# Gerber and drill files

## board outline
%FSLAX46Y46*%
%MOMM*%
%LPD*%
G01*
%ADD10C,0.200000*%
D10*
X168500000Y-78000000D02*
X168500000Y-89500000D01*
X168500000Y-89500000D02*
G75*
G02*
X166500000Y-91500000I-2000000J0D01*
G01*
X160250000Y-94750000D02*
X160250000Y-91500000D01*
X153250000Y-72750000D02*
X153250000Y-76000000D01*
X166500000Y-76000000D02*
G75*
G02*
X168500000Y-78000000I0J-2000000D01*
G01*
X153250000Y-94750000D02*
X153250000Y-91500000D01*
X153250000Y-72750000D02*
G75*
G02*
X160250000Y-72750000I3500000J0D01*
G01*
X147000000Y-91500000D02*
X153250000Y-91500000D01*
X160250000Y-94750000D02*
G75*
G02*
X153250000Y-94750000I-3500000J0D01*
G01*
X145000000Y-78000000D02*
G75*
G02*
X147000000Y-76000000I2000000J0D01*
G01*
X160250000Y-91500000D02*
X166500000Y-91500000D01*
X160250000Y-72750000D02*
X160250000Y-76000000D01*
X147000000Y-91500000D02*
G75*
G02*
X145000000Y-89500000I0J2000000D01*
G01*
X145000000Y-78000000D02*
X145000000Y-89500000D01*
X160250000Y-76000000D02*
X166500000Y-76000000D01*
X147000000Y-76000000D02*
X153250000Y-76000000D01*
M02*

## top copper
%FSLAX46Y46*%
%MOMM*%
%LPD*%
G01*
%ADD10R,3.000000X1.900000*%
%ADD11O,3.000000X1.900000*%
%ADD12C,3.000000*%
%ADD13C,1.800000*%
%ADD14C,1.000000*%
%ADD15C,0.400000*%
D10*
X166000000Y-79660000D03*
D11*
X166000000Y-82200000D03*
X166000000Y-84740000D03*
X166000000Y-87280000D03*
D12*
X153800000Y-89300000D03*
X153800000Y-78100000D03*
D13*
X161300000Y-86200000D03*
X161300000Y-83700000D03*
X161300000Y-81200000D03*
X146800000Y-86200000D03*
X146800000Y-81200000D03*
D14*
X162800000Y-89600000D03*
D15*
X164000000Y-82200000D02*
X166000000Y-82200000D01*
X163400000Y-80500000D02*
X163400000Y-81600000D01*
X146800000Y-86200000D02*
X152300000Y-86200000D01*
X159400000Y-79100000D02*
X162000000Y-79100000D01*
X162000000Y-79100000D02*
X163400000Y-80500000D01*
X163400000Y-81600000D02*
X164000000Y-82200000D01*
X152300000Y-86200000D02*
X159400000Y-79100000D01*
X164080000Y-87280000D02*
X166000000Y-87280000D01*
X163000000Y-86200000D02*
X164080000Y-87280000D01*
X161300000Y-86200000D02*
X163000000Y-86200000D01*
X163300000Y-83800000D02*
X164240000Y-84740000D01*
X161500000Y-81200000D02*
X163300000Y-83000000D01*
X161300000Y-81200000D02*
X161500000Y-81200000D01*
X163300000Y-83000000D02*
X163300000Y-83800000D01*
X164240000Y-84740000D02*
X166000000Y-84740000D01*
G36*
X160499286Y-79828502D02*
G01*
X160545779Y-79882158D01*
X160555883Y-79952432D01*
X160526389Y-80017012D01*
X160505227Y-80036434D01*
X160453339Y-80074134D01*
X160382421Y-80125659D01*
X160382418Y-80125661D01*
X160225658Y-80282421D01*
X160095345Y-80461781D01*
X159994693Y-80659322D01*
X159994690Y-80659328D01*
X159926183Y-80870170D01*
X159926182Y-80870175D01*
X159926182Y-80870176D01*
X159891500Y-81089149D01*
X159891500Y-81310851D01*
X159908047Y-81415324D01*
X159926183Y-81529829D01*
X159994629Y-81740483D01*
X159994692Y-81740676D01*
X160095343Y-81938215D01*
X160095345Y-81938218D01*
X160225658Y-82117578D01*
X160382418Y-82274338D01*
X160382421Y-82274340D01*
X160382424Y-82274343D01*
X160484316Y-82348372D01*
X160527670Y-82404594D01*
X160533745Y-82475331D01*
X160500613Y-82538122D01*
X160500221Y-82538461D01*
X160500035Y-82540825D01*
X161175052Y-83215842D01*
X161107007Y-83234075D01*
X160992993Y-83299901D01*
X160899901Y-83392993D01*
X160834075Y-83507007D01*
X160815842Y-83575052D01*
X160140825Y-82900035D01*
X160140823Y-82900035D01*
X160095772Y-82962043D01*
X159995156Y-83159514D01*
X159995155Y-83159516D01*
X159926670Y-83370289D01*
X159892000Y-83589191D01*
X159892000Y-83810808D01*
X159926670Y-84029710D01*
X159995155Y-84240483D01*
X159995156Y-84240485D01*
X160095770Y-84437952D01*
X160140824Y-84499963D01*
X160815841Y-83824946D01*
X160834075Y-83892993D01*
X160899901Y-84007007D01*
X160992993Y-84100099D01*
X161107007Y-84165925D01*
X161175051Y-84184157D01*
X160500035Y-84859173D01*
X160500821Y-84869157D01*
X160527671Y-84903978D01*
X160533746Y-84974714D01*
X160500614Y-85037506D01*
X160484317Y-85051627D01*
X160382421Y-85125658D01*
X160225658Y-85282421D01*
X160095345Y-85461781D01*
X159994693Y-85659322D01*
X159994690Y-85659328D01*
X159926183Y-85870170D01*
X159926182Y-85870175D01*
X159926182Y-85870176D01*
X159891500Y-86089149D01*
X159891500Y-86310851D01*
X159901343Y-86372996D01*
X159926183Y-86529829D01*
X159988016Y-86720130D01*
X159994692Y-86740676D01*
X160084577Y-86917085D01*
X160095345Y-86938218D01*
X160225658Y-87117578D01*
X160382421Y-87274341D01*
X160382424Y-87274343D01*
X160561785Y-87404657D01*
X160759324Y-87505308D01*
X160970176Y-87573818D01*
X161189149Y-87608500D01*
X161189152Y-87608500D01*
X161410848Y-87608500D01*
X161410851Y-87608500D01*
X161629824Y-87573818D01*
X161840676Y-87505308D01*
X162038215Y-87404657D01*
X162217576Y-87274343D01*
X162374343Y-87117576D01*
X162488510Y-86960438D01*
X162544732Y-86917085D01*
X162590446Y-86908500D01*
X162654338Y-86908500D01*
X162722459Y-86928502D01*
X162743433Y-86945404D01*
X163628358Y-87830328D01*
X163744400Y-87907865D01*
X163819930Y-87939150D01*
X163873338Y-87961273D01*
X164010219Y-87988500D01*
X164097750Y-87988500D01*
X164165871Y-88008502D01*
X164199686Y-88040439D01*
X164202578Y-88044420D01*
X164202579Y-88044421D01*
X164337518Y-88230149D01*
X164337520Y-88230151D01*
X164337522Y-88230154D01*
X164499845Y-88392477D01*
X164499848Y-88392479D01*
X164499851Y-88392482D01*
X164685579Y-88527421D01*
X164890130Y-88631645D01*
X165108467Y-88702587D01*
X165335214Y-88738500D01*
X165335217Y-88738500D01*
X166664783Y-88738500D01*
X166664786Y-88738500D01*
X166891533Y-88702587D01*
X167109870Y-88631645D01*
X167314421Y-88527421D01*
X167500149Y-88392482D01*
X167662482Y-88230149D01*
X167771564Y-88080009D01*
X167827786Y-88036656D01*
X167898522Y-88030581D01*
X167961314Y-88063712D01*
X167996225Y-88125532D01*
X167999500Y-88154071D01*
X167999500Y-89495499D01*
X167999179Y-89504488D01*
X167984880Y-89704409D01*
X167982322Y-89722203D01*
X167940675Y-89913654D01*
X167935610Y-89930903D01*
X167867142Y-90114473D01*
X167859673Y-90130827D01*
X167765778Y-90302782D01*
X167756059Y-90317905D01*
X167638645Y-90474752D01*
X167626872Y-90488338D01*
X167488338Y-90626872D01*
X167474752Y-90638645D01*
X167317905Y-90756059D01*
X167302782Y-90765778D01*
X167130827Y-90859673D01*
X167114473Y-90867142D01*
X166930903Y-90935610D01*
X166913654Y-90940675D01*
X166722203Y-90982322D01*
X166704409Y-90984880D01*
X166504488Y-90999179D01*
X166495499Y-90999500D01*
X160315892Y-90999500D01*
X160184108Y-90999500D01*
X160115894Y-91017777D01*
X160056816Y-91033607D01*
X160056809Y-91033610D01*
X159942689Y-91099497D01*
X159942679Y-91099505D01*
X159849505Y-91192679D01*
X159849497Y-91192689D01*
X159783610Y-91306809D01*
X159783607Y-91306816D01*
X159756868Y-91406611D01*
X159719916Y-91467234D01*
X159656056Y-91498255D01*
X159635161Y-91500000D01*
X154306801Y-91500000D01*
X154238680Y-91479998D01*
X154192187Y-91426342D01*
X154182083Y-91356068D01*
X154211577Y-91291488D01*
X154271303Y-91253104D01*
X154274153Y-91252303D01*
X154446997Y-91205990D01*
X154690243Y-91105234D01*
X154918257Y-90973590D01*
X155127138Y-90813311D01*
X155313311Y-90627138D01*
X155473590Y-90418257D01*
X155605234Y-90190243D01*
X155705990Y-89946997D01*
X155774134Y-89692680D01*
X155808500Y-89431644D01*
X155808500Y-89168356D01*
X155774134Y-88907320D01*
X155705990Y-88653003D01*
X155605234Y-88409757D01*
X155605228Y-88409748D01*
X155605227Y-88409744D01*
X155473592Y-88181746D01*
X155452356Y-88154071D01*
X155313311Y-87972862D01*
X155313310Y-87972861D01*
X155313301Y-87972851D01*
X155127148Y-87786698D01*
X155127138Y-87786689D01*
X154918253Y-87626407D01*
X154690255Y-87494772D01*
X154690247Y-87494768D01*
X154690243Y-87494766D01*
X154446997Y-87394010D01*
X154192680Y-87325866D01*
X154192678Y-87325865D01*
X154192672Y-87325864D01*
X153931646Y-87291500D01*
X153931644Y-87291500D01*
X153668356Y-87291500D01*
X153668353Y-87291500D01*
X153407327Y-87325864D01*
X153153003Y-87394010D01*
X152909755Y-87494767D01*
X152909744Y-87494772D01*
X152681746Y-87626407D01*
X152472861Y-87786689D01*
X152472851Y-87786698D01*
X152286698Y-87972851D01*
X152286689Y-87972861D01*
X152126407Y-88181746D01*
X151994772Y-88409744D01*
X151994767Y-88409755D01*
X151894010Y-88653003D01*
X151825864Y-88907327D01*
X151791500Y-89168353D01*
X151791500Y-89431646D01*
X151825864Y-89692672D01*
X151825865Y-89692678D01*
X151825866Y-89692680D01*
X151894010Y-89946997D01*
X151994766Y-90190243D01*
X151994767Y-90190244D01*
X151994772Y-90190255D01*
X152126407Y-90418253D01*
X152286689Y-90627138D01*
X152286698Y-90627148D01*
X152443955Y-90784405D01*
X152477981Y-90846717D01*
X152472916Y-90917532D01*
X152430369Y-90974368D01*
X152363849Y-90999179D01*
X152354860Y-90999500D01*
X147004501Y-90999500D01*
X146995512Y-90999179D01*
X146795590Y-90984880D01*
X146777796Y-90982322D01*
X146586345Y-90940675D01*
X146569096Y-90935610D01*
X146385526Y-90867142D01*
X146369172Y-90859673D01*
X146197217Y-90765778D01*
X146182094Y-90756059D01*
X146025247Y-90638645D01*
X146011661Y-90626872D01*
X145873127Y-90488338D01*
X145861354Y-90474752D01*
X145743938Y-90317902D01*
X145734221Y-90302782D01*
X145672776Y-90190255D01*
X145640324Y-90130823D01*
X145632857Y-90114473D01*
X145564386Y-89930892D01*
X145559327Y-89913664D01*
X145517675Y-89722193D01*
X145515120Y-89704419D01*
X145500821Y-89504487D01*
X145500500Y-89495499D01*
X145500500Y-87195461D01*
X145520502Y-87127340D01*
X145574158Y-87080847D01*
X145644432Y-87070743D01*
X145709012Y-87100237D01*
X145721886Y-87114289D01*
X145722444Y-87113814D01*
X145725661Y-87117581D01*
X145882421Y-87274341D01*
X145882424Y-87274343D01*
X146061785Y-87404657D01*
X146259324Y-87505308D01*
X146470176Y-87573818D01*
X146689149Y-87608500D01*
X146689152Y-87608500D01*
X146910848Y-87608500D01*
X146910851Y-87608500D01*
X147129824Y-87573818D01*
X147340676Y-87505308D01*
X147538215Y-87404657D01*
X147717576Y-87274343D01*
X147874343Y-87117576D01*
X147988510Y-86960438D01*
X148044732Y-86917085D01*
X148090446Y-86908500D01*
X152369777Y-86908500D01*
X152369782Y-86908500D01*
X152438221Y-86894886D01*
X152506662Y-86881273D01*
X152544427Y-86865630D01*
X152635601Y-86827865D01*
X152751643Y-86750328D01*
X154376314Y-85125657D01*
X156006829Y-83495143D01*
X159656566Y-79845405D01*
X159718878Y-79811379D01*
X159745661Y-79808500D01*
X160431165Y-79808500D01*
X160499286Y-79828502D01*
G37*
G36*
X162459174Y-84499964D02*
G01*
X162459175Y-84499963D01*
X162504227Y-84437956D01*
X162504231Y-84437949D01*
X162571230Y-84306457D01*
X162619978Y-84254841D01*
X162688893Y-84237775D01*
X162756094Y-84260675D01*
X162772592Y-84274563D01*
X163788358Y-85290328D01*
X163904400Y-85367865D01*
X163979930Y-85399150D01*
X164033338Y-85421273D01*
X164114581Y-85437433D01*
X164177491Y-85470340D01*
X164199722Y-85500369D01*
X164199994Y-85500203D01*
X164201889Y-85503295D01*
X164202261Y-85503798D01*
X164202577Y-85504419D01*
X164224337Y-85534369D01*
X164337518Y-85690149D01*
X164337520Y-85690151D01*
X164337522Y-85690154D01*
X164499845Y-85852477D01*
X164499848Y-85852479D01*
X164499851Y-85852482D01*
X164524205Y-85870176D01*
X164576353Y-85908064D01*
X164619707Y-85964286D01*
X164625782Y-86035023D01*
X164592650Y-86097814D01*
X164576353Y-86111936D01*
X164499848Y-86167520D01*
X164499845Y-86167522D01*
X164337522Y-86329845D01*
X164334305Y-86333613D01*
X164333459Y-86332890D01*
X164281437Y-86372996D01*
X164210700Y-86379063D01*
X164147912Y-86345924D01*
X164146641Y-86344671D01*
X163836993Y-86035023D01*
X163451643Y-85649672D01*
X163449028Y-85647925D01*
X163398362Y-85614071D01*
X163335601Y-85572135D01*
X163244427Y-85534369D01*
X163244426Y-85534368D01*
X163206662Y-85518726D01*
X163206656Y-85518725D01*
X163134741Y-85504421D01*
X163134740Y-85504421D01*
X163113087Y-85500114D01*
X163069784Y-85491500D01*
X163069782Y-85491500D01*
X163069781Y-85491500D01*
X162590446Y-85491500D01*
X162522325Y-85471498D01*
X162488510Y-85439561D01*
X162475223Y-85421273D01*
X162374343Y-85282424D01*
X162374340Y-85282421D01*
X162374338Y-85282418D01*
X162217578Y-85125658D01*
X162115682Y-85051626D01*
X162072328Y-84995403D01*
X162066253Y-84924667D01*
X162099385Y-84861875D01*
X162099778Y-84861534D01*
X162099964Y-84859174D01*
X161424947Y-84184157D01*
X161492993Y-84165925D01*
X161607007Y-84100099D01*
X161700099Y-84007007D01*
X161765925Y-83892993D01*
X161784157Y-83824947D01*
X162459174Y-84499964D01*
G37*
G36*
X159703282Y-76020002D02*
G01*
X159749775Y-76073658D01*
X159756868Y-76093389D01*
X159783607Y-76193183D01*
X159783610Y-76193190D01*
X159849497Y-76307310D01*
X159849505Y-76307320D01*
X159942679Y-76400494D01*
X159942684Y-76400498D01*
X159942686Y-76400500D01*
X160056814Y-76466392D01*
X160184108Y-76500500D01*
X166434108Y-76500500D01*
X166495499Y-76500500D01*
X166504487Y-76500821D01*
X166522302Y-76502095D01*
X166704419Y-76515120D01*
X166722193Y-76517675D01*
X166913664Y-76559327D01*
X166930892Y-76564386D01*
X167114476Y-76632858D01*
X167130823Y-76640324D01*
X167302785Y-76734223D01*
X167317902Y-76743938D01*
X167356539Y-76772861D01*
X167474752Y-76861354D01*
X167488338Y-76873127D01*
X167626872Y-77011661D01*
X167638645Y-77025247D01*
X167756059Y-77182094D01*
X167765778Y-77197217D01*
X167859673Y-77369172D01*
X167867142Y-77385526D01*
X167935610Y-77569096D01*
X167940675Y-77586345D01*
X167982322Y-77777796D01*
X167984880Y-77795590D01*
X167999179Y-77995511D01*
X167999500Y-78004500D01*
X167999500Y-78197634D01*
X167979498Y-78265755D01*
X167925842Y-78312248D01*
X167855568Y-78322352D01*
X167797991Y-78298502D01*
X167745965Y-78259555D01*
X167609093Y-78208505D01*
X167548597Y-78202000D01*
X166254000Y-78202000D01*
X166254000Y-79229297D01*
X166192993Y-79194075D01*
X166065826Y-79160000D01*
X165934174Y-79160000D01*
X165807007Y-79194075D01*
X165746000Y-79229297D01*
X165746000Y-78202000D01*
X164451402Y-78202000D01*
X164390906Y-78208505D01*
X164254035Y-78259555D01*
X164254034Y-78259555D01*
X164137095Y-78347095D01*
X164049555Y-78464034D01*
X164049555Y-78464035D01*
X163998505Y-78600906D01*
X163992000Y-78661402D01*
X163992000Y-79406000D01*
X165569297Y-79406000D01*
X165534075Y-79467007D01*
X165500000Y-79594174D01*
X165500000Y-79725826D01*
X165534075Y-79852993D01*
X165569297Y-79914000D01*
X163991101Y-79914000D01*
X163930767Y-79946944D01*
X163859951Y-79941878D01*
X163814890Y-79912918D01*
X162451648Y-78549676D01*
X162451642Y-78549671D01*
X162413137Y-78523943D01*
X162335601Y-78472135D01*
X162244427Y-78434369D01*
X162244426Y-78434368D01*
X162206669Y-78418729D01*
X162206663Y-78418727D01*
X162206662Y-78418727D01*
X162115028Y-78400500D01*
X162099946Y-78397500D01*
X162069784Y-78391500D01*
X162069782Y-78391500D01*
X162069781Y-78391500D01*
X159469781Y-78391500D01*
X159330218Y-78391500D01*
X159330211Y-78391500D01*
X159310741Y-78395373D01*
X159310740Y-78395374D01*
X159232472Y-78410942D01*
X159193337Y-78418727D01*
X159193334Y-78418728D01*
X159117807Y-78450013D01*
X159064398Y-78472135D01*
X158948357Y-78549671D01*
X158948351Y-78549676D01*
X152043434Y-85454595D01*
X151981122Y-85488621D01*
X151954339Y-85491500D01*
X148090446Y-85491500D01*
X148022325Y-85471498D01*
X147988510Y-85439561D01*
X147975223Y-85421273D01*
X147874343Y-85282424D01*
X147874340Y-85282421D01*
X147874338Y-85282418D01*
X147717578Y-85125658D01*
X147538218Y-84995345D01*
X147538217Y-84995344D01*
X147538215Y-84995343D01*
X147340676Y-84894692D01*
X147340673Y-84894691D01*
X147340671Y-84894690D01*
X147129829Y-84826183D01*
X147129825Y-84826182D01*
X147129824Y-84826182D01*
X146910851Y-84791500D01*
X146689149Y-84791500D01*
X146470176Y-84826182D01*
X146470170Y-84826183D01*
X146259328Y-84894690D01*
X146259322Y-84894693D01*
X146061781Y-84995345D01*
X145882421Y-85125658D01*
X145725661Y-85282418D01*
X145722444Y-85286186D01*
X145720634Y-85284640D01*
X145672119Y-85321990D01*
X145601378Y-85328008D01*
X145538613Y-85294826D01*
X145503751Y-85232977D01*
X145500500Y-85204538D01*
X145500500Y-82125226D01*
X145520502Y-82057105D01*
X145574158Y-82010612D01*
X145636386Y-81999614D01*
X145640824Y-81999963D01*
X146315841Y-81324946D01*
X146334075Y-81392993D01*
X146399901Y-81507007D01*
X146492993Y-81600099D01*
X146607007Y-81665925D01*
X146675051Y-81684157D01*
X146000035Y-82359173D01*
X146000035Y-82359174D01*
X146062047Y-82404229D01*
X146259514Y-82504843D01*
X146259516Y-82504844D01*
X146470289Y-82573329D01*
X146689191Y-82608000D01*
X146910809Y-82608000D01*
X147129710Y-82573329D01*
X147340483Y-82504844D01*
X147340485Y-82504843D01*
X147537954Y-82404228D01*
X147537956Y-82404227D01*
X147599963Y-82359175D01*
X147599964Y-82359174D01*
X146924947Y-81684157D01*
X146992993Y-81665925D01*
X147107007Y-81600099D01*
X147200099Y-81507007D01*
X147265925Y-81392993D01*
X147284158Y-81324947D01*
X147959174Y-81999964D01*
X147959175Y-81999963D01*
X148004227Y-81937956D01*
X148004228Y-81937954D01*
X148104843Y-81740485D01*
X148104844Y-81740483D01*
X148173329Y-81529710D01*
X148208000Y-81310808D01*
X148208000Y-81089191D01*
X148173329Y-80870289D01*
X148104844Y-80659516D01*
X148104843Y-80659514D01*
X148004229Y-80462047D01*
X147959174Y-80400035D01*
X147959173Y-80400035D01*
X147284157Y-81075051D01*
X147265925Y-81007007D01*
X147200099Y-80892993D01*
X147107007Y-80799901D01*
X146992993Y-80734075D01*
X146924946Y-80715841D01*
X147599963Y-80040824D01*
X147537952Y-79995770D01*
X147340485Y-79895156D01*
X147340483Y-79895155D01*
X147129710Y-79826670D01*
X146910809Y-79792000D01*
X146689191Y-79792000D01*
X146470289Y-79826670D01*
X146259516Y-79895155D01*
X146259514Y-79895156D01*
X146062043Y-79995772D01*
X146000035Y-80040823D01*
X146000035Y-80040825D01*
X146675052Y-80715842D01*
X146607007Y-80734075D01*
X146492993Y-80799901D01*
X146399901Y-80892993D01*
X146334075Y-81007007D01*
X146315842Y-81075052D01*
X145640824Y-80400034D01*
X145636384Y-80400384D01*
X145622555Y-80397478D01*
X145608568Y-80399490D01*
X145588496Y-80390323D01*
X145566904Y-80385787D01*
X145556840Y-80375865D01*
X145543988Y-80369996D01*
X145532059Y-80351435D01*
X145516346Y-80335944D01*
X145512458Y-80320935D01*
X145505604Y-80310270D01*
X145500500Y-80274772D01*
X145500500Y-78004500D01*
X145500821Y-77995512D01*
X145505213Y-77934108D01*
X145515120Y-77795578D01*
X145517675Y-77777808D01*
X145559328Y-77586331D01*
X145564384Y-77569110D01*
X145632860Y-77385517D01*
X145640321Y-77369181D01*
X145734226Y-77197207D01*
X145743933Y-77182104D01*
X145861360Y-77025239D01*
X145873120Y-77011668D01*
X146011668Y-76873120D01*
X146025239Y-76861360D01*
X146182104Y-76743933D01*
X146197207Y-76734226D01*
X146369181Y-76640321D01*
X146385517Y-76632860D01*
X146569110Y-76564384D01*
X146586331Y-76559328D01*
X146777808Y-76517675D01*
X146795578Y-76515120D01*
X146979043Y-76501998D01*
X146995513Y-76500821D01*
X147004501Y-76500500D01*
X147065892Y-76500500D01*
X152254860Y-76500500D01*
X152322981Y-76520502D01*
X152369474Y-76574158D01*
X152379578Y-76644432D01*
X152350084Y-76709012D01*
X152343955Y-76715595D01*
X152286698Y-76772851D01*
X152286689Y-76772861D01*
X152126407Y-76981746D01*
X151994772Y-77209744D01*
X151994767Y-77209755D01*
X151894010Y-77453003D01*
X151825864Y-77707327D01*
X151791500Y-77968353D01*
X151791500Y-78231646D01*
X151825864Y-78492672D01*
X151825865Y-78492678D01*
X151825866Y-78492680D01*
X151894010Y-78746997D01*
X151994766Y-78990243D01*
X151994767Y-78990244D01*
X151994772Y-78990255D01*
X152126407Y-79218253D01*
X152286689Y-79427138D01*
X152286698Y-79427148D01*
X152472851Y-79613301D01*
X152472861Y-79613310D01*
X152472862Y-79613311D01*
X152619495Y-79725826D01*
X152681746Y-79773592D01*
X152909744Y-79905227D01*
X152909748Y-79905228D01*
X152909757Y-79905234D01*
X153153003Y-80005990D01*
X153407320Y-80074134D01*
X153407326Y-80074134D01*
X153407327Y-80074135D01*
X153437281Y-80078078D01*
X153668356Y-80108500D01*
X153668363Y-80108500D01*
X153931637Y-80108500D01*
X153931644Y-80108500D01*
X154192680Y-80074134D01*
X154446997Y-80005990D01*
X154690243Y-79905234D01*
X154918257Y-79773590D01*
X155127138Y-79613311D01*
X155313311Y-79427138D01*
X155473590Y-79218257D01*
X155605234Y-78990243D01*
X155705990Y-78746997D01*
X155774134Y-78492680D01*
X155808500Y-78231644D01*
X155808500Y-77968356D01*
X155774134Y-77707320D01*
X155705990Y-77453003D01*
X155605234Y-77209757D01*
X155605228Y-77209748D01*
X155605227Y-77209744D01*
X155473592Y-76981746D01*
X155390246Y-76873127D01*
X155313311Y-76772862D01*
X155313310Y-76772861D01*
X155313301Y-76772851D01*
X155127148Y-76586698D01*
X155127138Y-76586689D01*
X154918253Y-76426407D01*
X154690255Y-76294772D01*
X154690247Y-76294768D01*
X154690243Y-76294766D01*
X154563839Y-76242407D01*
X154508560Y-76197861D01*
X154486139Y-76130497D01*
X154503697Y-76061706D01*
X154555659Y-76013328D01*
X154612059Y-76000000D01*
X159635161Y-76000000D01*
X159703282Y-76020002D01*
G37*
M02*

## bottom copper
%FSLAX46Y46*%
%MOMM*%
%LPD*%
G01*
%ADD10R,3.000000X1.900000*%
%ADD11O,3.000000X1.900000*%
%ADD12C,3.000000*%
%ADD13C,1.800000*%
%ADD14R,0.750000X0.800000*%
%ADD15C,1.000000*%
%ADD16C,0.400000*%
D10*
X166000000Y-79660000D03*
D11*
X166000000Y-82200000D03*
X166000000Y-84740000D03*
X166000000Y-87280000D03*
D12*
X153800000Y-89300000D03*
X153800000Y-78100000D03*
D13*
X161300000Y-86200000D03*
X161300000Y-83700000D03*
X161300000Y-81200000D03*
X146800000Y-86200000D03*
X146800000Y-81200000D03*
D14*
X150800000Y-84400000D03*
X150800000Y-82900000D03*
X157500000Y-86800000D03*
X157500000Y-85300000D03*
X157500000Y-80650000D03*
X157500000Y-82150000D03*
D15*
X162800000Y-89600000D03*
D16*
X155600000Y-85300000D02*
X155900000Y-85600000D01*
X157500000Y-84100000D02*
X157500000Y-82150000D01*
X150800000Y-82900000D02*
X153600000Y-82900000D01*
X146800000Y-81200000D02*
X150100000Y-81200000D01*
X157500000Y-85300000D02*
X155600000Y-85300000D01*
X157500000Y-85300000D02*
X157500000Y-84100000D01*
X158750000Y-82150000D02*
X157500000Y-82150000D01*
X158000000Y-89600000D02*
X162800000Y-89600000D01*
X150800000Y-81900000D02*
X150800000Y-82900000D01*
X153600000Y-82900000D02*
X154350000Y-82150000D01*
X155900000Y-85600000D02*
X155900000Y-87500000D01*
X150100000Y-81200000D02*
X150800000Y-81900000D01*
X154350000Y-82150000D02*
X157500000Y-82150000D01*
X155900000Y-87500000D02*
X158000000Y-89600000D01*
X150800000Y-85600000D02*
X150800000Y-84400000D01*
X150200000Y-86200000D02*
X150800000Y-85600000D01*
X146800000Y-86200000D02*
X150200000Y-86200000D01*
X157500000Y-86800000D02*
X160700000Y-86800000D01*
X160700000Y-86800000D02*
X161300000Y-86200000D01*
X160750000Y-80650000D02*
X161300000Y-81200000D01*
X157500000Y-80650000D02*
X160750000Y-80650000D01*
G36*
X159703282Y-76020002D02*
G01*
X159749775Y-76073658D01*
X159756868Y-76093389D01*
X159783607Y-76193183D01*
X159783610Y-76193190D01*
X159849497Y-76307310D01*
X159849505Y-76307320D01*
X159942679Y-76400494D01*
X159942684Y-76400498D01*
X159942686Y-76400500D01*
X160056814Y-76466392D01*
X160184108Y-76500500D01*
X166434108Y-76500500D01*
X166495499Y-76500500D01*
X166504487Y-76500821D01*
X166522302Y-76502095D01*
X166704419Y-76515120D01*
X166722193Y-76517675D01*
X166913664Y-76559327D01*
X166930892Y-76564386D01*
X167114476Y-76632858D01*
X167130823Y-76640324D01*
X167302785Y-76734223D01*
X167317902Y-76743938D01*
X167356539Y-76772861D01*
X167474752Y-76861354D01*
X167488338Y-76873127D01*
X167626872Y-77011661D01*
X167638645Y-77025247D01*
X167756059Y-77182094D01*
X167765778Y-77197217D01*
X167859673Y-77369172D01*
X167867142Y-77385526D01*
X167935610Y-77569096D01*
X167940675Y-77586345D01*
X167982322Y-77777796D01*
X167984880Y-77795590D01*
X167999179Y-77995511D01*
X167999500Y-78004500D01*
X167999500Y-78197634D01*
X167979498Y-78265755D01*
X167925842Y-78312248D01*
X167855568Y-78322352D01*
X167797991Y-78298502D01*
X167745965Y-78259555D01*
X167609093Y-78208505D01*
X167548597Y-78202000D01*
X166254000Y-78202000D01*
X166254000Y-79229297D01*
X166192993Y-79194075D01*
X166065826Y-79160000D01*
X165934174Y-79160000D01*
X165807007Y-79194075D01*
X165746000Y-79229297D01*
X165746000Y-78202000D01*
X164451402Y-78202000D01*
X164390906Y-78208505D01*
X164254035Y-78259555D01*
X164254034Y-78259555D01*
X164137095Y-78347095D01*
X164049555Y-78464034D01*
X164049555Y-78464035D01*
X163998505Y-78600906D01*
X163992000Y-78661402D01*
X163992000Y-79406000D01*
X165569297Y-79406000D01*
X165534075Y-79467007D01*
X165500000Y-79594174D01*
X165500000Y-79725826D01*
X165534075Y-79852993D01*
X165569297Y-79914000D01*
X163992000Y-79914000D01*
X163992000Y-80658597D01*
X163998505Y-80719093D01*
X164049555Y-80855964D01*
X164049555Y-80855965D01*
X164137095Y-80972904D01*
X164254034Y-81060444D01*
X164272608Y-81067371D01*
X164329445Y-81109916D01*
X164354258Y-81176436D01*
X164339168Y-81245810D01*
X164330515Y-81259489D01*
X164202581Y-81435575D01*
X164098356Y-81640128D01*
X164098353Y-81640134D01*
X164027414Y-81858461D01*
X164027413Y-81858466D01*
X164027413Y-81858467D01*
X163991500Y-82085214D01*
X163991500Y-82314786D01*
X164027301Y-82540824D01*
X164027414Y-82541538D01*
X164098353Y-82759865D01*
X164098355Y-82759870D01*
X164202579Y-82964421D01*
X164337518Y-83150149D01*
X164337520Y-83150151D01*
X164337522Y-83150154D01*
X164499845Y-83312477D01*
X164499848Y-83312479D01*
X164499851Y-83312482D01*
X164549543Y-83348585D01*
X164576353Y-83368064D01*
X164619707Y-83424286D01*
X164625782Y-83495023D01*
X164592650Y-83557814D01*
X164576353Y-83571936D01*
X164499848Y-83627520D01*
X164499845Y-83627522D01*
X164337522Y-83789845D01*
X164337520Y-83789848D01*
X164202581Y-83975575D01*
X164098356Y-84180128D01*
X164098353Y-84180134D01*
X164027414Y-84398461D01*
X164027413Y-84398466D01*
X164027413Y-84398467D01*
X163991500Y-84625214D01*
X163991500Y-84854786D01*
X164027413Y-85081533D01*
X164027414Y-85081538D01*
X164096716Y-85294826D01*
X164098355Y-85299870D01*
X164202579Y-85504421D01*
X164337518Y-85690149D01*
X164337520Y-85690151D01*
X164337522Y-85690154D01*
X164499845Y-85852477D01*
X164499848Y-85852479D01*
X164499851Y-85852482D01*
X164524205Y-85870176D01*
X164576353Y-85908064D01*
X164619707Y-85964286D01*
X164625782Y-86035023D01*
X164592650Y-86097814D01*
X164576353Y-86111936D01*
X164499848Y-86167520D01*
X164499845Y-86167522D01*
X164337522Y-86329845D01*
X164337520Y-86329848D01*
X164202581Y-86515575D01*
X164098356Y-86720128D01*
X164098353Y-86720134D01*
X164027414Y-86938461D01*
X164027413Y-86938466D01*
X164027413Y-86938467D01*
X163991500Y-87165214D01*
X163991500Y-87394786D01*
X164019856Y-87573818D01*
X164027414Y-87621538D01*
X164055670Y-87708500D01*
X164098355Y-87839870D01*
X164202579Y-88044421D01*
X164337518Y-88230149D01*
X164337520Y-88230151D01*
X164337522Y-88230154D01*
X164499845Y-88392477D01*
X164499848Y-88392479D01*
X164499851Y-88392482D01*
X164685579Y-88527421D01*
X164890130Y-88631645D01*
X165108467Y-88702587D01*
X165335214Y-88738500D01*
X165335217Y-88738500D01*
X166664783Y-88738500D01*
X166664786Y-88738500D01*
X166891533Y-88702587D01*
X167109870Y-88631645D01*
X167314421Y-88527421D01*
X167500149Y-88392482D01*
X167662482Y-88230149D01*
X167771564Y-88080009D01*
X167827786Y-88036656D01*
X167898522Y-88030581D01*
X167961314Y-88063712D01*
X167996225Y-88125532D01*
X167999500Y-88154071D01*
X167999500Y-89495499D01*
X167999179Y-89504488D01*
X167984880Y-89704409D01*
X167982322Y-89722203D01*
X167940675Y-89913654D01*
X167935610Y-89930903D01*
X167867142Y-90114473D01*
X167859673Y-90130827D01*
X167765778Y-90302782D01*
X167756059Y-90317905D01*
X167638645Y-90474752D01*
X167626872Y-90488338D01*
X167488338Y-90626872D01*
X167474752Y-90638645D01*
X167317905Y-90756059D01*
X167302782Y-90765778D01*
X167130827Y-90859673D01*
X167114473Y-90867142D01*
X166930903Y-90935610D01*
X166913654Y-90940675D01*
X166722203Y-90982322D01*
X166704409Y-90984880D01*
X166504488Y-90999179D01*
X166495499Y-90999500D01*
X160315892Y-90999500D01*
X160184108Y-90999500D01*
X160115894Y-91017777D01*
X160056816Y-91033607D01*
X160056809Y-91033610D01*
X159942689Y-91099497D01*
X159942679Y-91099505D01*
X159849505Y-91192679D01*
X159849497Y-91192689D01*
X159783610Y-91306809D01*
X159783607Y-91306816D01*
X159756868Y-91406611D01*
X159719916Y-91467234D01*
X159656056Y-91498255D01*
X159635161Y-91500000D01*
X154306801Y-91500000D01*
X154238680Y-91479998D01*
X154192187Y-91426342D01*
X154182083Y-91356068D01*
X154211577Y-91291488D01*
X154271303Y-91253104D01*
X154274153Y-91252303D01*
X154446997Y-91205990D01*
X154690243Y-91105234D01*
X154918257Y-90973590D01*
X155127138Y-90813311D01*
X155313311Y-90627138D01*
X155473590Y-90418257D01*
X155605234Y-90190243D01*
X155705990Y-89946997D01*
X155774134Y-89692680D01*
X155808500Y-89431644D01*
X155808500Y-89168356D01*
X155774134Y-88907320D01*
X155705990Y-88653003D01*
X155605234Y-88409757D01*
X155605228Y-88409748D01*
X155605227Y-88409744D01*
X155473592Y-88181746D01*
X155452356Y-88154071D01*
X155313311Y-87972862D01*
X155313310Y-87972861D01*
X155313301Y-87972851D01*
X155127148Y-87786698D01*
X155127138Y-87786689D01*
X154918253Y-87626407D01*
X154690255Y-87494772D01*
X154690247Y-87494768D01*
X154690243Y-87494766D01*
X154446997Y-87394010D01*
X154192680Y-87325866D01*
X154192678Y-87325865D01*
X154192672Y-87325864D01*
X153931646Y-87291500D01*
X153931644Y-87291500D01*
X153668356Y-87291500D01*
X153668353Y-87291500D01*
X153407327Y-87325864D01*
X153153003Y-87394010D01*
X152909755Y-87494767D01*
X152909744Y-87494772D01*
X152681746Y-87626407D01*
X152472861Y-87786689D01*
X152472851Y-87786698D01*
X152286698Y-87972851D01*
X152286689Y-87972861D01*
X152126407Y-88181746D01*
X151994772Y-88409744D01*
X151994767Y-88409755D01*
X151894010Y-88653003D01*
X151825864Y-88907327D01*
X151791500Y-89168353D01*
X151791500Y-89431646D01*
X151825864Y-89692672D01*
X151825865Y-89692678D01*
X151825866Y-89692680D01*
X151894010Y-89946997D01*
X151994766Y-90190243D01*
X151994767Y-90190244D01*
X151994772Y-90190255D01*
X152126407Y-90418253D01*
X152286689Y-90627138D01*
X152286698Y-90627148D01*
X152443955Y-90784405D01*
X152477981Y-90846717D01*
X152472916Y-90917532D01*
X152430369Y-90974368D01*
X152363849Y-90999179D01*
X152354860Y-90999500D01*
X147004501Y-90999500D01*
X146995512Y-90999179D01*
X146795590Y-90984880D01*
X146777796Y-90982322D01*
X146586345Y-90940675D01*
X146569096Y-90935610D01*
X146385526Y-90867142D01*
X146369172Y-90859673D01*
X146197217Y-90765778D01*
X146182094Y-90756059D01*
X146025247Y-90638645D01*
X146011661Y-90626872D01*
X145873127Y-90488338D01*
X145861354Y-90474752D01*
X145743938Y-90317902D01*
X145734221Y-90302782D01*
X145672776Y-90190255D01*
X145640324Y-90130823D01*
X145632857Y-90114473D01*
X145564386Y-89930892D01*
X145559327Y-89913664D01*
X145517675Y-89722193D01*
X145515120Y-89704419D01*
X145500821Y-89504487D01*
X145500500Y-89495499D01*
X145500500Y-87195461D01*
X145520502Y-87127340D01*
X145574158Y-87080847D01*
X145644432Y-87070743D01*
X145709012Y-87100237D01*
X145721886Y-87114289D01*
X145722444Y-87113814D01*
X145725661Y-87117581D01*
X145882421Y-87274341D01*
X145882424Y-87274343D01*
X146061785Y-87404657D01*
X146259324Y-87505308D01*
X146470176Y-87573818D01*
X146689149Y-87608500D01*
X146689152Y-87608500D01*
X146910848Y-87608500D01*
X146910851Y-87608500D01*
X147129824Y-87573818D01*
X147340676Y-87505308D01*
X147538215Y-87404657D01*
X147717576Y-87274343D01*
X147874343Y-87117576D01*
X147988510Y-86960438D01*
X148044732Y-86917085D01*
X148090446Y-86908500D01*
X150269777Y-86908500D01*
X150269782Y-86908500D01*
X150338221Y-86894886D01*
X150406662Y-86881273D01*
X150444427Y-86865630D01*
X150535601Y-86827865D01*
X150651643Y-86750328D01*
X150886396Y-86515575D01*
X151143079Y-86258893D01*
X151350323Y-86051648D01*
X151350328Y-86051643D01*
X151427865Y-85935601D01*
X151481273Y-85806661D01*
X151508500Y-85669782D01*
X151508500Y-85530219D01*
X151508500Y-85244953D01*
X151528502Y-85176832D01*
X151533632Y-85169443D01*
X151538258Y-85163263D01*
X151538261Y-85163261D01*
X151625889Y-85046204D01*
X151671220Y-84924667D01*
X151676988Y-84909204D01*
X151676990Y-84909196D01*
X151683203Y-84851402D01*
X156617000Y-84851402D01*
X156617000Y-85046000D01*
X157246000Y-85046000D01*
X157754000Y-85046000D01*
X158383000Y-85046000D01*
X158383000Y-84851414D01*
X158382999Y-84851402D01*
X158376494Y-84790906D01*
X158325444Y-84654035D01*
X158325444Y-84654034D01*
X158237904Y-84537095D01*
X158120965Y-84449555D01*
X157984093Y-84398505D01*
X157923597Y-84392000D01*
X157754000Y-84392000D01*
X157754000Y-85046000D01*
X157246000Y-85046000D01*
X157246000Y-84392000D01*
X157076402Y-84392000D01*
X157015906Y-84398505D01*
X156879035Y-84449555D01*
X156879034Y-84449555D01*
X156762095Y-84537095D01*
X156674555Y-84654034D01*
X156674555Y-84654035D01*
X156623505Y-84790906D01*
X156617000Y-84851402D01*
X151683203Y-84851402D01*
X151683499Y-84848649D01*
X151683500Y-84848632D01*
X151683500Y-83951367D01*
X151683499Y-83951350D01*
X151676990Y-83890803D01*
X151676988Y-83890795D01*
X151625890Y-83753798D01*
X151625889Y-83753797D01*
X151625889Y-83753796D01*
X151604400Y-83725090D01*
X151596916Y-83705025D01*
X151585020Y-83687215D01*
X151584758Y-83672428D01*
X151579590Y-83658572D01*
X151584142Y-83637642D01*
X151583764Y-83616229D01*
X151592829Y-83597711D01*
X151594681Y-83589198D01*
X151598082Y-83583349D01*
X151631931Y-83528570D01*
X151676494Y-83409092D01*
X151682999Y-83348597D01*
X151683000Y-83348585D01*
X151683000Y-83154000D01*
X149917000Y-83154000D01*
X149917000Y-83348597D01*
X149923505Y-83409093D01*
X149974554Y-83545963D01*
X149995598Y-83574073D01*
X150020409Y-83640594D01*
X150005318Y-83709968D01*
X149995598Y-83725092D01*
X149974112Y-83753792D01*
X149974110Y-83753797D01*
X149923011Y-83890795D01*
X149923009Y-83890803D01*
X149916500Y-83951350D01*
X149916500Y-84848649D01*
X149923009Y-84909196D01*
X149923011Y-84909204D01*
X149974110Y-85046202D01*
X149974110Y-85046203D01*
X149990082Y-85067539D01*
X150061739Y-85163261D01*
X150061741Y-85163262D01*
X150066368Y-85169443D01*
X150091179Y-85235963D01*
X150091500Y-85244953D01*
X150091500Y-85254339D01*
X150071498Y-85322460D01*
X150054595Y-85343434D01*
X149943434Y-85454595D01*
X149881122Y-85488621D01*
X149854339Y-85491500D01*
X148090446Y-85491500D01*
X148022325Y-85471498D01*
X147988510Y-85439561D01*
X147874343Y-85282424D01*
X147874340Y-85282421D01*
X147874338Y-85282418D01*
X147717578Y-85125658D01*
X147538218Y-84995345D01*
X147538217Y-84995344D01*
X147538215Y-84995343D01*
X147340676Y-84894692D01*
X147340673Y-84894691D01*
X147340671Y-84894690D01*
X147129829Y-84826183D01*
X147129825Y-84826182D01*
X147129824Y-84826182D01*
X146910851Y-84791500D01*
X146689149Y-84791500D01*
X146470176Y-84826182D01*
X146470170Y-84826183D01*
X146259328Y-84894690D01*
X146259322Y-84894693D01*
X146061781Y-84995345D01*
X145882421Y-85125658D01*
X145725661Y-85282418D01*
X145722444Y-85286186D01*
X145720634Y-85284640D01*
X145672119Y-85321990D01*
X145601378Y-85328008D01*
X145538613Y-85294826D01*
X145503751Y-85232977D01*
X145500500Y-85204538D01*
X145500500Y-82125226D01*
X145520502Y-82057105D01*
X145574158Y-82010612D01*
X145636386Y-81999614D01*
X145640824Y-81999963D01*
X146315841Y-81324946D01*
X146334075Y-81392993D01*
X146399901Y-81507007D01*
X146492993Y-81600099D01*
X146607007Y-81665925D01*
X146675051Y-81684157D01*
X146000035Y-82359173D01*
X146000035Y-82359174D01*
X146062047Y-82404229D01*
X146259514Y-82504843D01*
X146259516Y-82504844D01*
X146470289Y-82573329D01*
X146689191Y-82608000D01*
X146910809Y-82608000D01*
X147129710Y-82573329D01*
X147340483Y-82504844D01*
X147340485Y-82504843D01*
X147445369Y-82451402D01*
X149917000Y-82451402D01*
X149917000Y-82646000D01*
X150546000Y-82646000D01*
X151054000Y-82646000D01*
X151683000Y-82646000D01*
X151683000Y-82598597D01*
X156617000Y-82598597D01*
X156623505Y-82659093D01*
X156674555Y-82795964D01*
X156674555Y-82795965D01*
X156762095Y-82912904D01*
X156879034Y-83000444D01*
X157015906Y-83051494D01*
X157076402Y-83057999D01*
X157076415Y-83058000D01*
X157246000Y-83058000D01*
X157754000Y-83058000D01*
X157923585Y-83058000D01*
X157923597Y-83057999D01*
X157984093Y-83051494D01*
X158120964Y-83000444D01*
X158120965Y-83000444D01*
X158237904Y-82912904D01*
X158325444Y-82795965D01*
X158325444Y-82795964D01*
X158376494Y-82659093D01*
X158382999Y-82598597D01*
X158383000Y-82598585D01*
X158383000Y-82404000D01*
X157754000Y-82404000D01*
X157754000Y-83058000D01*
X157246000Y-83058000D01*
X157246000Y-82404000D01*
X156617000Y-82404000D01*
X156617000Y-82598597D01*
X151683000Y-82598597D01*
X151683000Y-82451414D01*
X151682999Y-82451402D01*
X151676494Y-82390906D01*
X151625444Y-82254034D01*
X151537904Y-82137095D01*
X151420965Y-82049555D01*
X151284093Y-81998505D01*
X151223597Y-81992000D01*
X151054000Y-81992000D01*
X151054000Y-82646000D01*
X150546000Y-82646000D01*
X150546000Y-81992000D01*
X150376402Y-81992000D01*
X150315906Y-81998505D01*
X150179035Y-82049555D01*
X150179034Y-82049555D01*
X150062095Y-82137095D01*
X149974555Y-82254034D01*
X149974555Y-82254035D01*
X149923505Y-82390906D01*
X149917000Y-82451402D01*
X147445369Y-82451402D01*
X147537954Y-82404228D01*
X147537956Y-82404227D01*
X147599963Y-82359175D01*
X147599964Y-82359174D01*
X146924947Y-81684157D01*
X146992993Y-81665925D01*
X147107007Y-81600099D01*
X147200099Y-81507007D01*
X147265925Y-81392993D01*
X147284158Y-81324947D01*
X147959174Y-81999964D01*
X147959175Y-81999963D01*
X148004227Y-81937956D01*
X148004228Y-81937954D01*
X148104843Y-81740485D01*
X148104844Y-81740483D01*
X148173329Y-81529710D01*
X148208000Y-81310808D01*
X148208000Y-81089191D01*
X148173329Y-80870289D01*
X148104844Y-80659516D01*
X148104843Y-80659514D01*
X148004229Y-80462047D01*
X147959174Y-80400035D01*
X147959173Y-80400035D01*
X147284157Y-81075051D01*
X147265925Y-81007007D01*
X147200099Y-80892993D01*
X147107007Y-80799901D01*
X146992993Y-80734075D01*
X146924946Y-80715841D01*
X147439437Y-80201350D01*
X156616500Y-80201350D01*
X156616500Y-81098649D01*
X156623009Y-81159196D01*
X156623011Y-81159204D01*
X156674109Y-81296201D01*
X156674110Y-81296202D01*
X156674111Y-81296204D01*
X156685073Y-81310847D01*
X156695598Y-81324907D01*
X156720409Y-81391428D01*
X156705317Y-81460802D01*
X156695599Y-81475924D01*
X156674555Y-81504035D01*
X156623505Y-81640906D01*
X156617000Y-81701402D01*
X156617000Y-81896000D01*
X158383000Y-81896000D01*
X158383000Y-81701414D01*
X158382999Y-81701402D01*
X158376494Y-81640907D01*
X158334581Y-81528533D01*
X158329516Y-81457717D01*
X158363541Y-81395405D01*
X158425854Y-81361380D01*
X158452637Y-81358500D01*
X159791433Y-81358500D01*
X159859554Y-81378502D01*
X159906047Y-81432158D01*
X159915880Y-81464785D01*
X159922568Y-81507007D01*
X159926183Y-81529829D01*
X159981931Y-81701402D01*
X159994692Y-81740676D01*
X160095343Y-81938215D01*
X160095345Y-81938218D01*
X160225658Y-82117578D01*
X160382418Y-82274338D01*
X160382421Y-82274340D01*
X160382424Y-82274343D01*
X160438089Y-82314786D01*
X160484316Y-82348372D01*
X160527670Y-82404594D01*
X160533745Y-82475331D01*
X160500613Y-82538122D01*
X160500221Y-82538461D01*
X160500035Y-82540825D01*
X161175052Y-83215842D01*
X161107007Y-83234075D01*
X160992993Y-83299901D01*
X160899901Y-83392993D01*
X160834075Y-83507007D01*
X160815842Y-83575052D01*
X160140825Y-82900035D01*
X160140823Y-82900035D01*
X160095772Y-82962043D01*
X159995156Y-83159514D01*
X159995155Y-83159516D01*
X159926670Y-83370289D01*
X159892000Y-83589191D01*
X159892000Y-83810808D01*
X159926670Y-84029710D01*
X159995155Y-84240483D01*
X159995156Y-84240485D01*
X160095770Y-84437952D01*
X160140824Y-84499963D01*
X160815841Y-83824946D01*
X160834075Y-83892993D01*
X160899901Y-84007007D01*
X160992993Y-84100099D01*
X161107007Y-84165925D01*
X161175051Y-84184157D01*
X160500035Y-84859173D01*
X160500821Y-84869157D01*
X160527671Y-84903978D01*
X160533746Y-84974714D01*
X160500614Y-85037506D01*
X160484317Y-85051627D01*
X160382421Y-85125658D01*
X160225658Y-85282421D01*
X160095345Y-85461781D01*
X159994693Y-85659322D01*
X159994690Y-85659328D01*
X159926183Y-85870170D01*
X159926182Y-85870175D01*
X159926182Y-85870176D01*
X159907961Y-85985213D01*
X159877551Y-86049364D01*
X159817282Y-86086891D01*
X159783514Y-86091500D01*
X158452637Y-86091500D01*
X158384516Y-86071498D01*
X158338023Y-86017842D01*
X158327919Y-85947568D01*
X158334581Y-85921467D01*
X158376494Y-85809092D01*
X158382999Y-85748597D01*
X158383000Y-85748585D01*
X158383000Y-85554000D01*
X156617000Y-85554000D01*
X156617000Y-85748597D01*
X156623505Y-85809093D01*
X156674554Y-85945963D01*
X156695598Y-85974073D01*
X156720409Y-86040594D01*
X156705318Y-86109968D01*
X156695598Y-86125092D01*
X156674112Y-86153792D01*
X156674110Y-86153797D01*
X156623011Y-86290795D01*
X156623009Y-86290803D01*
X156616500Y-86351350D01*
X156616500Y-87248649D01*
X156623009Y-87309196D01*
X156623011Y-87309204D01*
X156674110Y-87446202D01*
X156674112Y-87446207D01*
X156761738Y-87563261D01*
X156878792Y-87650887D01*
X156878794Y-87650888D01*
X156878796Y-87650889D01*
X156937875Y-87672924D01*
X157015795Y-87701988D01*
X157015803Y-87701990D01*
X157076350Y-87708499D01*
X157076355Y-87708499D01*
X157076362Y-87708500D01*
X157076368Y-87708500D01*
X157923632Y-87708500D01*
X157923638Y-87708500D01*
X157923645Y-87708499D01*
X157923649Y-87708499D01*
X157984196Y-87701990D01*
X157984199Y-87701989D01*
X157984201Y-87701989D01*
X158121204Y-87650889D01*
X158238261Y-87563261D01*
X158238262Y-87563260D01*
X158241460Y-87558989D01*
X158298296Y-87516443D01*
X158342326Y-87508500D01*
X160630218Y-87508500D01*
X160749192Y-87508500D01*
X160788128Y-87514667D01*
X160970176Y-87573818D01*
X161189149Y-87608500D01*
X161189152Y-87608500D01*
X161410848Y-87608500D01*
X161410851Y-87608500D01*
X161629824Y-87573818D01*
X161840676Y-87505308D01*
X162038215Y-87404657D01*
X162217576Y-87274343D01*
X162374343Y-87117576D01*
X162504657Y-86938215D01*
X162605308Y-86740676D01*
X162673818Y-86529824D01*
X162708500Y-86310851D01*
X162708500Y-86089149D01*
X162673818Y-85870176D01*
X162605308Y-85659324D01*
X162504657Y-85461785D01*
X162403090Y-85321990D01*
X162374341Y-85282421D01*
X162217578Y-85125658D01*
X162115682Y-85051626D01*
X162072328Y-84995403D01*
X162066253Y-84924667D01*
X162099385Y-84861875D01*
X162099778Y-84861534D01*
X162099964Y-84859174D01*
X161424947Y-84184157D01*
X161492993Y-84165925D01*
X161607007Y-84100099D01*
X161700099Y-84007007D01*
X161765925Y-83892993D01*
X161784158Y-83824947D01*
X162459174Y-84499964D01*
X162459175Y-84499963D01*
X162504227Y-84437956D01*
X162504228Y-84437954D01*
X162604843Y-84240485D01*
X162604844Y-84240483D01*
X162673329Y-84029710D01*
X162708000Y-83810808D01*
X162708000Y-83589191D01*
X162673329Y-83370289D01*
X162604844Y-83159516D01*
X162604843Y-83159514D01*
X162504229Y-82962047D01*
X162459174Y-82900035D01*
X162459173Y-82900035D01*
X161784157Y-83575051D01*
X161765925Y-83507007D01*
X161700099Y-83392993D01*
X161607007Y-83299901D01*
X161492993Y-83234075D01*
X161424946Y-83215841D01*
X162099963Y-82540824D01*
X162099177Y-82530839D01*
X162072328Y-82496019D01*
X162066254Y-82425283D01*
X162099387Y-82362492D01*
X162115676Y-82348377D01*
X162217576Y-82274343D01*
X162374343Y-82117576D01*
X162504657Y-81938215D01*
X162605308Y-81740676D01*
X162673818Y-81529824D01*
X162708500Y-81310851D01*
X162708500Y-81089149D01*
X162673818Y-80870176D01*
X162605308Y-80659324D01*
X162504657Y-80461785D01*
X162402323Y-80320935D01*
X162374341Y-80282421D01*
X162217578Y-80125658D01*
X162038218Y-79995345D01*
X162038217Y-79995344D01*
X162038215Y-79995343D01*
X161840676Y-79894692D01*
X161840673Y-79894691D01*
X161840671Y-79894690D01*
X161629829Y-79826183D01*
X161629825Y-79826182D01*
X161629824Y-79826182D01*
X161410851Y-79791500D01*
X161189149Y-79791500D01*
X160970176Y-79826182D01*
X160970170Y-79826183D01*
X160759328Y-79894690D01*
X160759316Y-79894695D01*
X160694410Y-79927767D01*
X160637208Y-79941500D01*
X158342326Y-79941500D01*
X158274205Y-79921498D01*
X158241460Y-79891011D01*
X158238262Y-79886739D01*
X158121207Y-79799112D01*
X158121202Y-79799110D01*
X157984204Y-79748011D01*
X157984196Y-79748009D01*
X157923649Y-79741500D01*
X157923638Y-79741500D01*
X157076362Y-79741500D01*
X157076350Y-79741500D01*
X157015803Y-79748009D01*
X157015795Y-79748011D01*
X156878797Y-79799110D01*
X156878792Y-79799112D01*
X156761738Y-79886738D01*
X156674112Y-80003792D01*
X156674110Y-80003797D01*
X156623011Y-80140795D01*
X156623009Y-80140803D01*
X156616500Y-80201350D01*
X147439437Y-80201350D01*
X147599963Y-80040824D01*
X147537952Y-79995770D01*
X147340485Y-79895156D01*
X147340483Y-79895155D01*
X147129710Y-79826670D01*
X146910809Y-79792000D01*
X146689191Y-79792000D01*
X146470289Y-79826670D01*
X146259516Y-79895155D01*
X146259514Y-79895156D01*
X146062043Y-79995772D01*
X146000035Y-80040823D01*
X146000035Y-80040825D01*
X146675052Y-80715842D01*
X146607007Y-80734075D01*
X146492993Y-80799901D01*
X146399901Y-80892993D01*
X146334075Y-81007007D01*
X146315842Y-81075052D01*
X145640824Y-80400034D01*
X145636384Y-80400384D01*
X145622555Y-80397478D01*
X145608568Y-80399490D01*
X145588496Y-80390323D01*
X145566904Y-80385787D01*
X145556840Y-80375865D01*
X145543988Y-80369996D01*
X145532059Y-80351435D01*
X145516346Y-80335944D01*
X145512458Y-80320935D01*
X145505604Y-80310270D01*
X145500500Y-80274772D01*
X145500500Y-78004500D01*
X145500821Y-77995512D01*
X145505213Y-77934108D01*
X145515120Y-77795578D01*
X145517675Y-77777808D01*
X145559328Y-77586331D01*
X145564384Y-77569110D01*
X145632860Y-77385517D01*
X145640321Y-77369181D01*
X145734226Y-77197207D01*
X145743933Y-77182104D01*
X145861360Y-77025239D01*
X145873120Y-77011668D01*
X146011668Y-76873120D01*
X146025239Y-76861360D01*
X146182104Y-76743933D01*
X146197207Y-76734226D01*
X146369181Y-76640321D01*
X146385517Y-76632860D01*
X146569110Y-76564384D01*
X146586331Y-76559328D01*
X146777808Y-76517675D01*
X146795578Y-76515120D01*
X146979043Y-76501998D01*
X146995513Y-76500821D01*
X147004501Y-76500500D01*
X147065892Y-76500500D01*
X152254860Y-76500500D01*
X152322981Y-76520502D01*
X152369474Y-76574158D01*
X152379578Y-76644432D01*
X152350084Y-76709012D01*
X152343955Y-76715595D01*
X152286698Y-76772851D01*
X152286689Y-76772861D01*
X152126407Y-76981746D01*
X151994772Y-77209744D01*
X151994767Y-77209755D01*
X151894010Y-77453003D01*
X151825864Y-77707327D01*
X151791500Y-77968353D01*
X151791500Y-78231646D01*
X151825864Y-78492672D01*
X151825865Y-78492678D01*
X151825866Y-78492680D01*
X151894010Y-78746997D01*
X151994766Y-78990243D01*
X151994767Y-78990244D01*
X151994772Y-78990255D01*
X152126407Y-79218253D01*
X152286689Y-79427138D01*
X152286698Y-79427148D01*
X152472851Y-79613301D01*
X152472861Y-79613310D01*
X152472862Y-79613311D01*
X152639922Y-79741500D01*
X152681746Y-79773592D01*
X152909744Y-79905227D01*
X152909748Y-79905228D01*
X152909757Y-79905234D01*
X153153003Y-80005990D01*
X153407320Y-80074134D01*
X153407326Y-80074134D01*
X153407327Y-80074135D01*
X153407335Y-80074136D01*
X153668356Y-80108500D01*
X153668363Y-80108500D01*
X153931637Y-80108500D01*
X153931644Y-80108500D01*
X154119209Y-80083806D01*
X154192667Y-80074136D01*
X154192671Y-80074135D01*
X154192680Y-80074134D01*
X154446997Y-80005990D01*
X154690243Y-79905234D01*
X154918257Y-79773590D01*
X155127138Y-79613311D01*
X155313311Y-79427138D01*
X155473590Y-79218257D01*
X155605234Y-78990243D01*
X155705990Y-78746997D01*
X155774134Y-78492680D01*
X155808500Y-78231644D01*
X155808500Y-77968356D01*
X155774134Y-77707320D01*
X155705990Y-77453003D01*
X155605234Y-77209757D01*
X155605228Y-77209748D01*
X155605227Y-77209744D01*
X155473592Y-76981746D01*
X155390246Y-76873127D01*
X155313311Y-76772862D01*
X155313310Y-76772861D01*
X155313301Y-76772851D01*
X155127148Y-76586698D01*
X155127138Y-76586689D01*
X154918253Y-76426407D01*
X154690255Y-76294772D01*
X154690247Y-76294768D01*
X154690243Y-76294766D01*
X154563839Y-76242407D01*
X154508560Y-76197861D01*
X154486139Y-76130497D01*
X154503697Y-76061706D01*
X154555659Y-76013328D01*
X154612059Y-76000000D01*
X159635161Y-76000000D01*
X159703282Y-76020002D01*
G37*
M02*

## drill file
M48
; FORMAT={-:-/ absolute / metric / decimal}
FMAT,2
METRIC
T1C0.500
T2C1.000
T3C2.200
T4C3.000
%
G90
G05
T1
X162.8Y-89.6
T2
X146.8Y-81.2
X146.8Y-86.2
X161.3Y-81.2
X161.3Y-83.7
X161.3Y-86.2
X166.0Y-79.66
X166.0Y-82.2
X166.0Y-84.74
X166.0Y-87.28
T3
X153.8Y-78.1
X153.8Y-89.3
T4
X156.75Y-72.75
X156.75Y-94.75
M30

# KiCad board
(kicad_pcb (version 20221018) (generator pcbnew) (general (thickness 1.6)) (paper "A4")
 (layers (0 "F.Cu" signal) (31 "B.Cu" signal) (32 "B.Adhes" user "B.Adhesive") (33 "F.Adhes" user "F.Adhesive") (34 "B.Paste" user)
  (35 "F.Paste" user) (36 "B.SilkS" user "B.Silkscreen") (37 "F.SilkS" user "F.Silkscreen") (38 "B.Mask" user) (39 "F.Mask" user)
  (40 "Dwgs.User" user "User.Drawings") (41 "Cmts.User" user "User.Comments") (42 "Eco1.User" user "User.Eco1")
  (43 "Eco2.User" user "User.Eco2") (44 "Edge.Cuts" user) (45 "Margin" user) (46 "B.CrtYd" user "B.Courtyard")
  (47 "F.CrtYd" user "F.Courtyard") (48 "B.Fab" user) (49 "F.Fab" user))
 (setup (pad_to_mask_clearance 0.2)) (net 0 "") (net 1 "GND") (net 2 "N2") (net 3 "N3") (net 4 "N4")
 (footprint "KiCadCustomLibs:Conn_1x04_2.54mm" (layer "F.Cu") (at 166 79.66)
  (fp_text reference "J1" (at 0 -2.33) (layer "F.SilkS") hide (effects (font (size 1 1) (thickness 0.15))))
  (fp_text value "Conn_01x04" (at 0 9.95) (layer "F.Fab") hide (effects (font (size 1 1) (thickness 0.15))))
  (pad "1" thru_hole rect (at 0 0) (size 3 1.9) (drill 1) (layers "*.Cu" "*.Mask") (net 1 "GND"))
  (pad "2" thru_hole oval (at 0 2.54) (size 3 1.9) (drill 1) (layers "*.Cu" "*.Mask") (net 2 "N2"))
  (pad "3" thru_hole oval (at 0 5.08) (size 3 1.9) (drill 1) (layers "*.Cu" "*.Mask") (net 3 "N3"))
  (pad "4" thru_hole oval (at 0 7.62) (size 3 1.9) (drill 1) (layers "*.Cu" "*.Mask") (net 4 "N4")))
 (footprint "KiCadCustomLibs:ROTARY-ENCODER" (layer "F.Cu") (at 153.8 83.7 90)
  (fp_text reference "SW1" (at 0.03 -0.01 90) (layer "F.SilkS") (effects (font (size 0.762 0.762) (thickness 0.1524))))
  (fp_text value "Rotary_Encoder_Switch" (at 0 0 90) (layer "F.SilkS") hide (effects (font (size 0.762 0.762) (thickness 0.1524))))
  (pad "" thru_hole circle (at -5.6 0 90) (size 3 3) (drill 2.2) (layers "*.Cu" "*.Mask" "F.SilkS"))
  (pad "" thru_hole circle (at 5.6 0 90) (size 3 3) (drill 2.2) (layers "*.Cu" "*.Mask" "F.SilkS"))
  (pad "1" thru_hole circle (at -2.5 7.5 90) (size 1.8 1.8) (drill 1) (layers "*.Cu" "*.Mask" "F.SilkS") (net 4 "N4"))
  (pad "2" thru_hole circle (at 0 7.5 90) (size 1.8 1.8) (drill 1) (layers "*.Cu" "*.Mask" "F.SilkS") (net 1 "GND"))
  (pad "3" thru_hole circle (at 2.5 7.5 90) (size 1.8 1.8) (drill 1) (layers "*.Cu" "*.Mask" "F.SilkS") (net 3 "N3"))
  (pad "4" thru_hole circle (at -2.5 -7 90) (size 1.8 1.8) (drill 1) (layers "*.Cu" "*.Mask" "F.SilkS") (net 2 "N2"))
  (pad "5" thru_hole circle (at 2.5 -7 90) (size 1.8 1.8) (drill 1) (layers "*.Cu" "*.Mask" "F.SilkS") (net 1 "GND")))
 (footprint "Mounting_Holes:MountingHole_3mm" (layer "F.Cu") (at 156.75 72.75)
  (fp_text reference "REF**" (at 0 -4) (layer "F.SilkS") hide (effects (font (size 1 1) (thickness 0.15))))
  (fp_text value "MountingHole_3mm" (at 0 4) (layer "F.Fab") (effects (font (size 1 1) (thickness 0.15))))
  (pad "" np_thru_hole circle (at 0 0) (size 3 3) (drill 3) (layers "*.Cu" "*.Mask")))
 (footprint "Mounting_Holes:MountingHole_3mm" (layer "F.Cu") (at 156.75 94.75)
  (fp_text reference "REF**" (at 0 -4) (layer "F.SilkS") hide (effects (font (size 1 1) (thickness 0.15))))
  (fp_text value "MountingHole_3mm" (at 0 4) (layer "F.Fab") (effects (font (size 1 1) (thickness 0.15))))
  (pad "" np_thru_hole circle (at 0 0) (size 3 3) (drill 3) (layers "*.Cu" "*.Mask")))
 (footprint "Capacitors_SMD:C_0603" (layer "B.Cu") (at 150.8 83.65 90)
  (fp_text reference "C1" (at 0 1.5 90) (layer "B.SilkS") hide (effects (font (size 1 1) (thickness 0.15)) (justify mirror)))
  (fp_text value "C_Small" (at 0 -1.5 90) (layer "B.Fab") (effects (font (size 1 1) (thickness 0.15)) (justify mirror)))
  (pad "1" smd rect (at -0.75 0 90) (size 0.8 0.75) (layers "B.Cu" "B.Paste" "B.Mask") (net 2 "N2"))
  (pad "2" smd rect (at 0.75 0 90) (size 0.8 0.75) (layers "B.Cu" "B.Paste" "B.Mask") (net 1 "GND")))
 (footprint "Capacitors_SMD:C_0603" (layer "B.Cu") (at 157.5 86.05 90)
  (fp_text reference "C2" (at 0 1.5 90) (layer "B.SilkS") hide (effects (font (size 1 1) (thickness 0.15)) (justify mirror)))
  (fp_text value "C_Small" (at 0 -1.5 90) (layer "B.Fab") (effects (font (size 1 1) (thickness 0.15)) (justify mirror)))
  (pad "1" smd rect (at -0.75 0 90) (size 0.8 0.75) (layers "B.Cu" "B.Paste" "B.Mask") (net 4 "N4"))
  (pad "2" smd rect (at 0.75 0 90) (size 0.8 0.75) (layers "B.Cu" "B.Paste" "B.Mask") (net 1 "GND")))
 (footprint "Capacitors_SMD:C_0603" (layer "B.Cu") (at 157.5 81.4 -90)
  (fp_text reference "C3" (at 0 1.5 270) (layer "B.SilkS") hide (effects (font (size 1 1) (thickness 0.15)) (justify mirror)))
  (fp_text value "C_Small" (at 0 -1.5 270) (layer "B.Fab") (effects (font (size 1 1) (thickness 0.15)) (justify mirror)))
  (pad "1" smd rect (at -0.75 0 270) (size 0.8 0.75) (layers "B.Cu" "B.Paste" "B.Mask") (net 3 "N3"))
  (pad "2" smd rect (at 0.75 0 270) (size 0.8 0.75) (layers "B.Cu" "B.Paste" "B.Mask") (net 1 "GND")))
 (gr_line (start 168.5 78) (end 168.5 89.5) (stroke (width 0.2) (type solid)) (layer "Edge.Cuts"))
 (gr_arc (start 168.5 89.5) (mid 167.914214 90.914214) (end 166.5 91.5) (stroke (width 0.2) (type solid)) (layer "Edge.Cuts"))
 (gr_line (start 160.25 94.75) (end 160.25 91.5) (stroke (width 0.2) (type solid)) (layer "Edge.Cuts"))
 (gr_line (start 153.25 72.75) (end 153.25 76) (stroke (width 0.2) (type solid)) (layer "Edge.Cuts"))
 (gr_arc (start 166.5 76) (mid 167.914214 76.585786) (end 168.5 78) (stroke (width 0.2) (type solid)) (layer "Edge.Cuts"))
 (gr_line (start 153.25 94.75) (end 153.25 91.5) (stroke (width 0.2) (type solid)) (layer "Edge.Cuts"))
 (gr_arc (start 153.25 72.75) (mid 156.75 69.25) (end 160.25 72.75) (stroke (width 0.2) (type solid)) (layer "Edge.Cuts"))
 (gr_line (start 147 91.5) (end 153.25 91.5) (stroke (width 0.2) (type solid)) (layer "Edge.Cuts"))
 (gr_arc (start 160.25 94.75) (mid 156.75 98.25) (end 153.25 94.75) (stroke (width 0.2) (type solid)) (layer "Edge.Cuts"))
 (gr_arc (start 145 78) (mid 145.585786 76.585786) (end 147 76) (stroke (width 0.2) (type solid)) (layer "Edge.Cuts"))
 (gr_line (start 160.25 91.5) (end 166.5 91.5) (stroke (width 0.2) (type solid)) (layer "Edge.Cuts"))
 (gr_line (start 160.25 72.75) (end 160.25 76) (stroke (width 0.2) (type solid)) (layer "Edge.Cuts"))
 (gr_arc (start 147 91.5) (mid 145.585786 90.914214) (end 145 89.5) (stroke (width 0.2) (type solid)) (layer "Edge.Cuts"))
 (gr_line (start 145 78) (end 145 89.5) (stroke (width 0.2) (type solid)) (layer "Edge.Cuts"))
 (gr_line (start 160.25 76) (end 166.5 76) (stroke (width 0.2) (type solid)) (layer "Edge.Cuts"))
 (gr_line (start 147 76) (end 153.25 76) (stroke (width 0.2) (type solid)) (layer "Edge.Cuts"))
 (via (at 162.8 89.6) (size 1) (drill 0.5) (layers "F.Cu" "B.Cu") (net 1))
 (segment (start 155.6 85.3) (end 155.9 85.6) (width 0.4) (layer "B.Cu") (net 1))
 (segment (start 157.5 84.1) (end 157.5 82.15) (width 0.4) (layer "B.Cu") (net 1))
 (segment (start 150.8 82.9) (end 153.6 82.9) (width 0.4) (layer "B.Cu") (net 1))
 (segment (start 146.8 81.2) (end 150.1 81.2) (width 0.4) (layer "B.Cu") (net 1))
 (segment (start 157.5 85.3) (end 155.6 85.3) (width 0.4) (layer "B.Cu") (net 1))
 (segment (start 157.5 85.3) (end 157.5 84.1) (width 0.4) (layer "B.Cu") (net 1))
 (segment (start 158.75 82.15) (end 157.5 82.15) (width 0.4) (layer "B.Cu") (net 1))
 (segment (start 158 89.6) (end 162.8 89.6) (width 0.4) (layer "B.Cu") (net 1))
 (segment (start 150.8 81.9) (end 150.8 82.9) (width 0.4) (layer "B.Cu") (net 1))
 (segment (start 153.6 82.9) (end 154.35 82.15) (width 0.4) (layer "B.Cu") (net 1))
 (segment (start 155.9 85.6) (end 155.9 87.5) (width 0.4) (layer "B.Cu") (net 1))
 (segment (start 150.1 81.2) (end 150.8 81.9) (width 0.4) (layer "B.Cu") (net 1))
 (segment (start 154.35 82.15) (end 157.5 82.15) (width 0.4) (layer "B.Cu") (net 1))
 (segment (start 155.9 87.5) (end 158 89.6) (width 0.4) (layer "B.Cu") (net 1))
 (segment (start 164 82.2) (end 166 82.2) (width 0.4) (layer "F.Cu") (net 2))
 (segment (start 163.4 80.5) (end 163.4 81.6) (width 0.4) (layer "F.Cu") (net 2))
 (segment (start 146.8 86.2) (end 152.3 86.2) (width 0.4) (layer "F.Cu") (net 2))
 (segment (start 159.4 79.1) (end 162 79.1) (width 0.4) (layer "F.Cu") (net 2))
 (segment (start 162 79.1) (end 163.4 80.5) (width 0.4) (layer "F.Cu") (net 2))
 (segment (start 163.4 81.6) (end 164 82.2) (width 0.4) (layer "F.Cu") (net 2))
 (segment (start 152.3 86.2) (end 159.4 79.1) (width 0.4) (layer "F.Cu") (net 2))
 (segment (start 150.8 85.6) (end 150.8 84.4) (width 0.4) (layer "B.Cu") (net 2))
 (segment (start 150.2 86.2) (end 150.8 85.6) (width 0.4) (layer "B.Cu") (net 2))
 (segment (start 146.8 86.2) (end 150.2 86.2) (width 0.4) (layer "B.Cu") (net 2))
 (segment (start 164.08 87.28) (end 166 87.28) (width 0.4) (layer "F.Cu") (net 4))
 (segment (start 163 86.2) (end 164.08 87.28) (width 0.4) (layer "F.Cu") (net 4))
 (segment (start 161.3 86.2) (end 163 86.2) (width 0.4) (layer "F.Cu") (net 4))
 (segment (start 157.5 86.8) (end 160.7 86.8) (width 0.4) (layer "B.Cu") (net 4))
 (segment (start 160.7 86.8) (end 161.3 86.2) (width 0.4) (layer "B.Cu") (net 4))
 (segment (start 163.3 83.8) (end 164.24 84.74) (width 0.4) (layer "F.Cu") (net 3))
 (segment (start 161.5 81.2) (end 163.3 83) (width 0.4) (layer "F.Cu") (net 3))
 (segment (start 161.3 81.2) (end 161.5 81.2) (width 0.4) (layer "F.Cu") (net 3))
 (segment (start 163.3 83) (end 163.3 83.8) (width 0.4) (layer "F.Cu") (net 3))
 (segment (start 164.24 84.74) (end 166 84.74) (width 0.4) (layer "F.Cu") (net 3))
 (segment (start 160.75 80.65) (end 161.3 81.2) (width 0.4) (layer "B.Cu") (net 3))
 (segment (start 157.5 80.65) (end 160.75 80.65) (width 0.4) (layer "B.Cu") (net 3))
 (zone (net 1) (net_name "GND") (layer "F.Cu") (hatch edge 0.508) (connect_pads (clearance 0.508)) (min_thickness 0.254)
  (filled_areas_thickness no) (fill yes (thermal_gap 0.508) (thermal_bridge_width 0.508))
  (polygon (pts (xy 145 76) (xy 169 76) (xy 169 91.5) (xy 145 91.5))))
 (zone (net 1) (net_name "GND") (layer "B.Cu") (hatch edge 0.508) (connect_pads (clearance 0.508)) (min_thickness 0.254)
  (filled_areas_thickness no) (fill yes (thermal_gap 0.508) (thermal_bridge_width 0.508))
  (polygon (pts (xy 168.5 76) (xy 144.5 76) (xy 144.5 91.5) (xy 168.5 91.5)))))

